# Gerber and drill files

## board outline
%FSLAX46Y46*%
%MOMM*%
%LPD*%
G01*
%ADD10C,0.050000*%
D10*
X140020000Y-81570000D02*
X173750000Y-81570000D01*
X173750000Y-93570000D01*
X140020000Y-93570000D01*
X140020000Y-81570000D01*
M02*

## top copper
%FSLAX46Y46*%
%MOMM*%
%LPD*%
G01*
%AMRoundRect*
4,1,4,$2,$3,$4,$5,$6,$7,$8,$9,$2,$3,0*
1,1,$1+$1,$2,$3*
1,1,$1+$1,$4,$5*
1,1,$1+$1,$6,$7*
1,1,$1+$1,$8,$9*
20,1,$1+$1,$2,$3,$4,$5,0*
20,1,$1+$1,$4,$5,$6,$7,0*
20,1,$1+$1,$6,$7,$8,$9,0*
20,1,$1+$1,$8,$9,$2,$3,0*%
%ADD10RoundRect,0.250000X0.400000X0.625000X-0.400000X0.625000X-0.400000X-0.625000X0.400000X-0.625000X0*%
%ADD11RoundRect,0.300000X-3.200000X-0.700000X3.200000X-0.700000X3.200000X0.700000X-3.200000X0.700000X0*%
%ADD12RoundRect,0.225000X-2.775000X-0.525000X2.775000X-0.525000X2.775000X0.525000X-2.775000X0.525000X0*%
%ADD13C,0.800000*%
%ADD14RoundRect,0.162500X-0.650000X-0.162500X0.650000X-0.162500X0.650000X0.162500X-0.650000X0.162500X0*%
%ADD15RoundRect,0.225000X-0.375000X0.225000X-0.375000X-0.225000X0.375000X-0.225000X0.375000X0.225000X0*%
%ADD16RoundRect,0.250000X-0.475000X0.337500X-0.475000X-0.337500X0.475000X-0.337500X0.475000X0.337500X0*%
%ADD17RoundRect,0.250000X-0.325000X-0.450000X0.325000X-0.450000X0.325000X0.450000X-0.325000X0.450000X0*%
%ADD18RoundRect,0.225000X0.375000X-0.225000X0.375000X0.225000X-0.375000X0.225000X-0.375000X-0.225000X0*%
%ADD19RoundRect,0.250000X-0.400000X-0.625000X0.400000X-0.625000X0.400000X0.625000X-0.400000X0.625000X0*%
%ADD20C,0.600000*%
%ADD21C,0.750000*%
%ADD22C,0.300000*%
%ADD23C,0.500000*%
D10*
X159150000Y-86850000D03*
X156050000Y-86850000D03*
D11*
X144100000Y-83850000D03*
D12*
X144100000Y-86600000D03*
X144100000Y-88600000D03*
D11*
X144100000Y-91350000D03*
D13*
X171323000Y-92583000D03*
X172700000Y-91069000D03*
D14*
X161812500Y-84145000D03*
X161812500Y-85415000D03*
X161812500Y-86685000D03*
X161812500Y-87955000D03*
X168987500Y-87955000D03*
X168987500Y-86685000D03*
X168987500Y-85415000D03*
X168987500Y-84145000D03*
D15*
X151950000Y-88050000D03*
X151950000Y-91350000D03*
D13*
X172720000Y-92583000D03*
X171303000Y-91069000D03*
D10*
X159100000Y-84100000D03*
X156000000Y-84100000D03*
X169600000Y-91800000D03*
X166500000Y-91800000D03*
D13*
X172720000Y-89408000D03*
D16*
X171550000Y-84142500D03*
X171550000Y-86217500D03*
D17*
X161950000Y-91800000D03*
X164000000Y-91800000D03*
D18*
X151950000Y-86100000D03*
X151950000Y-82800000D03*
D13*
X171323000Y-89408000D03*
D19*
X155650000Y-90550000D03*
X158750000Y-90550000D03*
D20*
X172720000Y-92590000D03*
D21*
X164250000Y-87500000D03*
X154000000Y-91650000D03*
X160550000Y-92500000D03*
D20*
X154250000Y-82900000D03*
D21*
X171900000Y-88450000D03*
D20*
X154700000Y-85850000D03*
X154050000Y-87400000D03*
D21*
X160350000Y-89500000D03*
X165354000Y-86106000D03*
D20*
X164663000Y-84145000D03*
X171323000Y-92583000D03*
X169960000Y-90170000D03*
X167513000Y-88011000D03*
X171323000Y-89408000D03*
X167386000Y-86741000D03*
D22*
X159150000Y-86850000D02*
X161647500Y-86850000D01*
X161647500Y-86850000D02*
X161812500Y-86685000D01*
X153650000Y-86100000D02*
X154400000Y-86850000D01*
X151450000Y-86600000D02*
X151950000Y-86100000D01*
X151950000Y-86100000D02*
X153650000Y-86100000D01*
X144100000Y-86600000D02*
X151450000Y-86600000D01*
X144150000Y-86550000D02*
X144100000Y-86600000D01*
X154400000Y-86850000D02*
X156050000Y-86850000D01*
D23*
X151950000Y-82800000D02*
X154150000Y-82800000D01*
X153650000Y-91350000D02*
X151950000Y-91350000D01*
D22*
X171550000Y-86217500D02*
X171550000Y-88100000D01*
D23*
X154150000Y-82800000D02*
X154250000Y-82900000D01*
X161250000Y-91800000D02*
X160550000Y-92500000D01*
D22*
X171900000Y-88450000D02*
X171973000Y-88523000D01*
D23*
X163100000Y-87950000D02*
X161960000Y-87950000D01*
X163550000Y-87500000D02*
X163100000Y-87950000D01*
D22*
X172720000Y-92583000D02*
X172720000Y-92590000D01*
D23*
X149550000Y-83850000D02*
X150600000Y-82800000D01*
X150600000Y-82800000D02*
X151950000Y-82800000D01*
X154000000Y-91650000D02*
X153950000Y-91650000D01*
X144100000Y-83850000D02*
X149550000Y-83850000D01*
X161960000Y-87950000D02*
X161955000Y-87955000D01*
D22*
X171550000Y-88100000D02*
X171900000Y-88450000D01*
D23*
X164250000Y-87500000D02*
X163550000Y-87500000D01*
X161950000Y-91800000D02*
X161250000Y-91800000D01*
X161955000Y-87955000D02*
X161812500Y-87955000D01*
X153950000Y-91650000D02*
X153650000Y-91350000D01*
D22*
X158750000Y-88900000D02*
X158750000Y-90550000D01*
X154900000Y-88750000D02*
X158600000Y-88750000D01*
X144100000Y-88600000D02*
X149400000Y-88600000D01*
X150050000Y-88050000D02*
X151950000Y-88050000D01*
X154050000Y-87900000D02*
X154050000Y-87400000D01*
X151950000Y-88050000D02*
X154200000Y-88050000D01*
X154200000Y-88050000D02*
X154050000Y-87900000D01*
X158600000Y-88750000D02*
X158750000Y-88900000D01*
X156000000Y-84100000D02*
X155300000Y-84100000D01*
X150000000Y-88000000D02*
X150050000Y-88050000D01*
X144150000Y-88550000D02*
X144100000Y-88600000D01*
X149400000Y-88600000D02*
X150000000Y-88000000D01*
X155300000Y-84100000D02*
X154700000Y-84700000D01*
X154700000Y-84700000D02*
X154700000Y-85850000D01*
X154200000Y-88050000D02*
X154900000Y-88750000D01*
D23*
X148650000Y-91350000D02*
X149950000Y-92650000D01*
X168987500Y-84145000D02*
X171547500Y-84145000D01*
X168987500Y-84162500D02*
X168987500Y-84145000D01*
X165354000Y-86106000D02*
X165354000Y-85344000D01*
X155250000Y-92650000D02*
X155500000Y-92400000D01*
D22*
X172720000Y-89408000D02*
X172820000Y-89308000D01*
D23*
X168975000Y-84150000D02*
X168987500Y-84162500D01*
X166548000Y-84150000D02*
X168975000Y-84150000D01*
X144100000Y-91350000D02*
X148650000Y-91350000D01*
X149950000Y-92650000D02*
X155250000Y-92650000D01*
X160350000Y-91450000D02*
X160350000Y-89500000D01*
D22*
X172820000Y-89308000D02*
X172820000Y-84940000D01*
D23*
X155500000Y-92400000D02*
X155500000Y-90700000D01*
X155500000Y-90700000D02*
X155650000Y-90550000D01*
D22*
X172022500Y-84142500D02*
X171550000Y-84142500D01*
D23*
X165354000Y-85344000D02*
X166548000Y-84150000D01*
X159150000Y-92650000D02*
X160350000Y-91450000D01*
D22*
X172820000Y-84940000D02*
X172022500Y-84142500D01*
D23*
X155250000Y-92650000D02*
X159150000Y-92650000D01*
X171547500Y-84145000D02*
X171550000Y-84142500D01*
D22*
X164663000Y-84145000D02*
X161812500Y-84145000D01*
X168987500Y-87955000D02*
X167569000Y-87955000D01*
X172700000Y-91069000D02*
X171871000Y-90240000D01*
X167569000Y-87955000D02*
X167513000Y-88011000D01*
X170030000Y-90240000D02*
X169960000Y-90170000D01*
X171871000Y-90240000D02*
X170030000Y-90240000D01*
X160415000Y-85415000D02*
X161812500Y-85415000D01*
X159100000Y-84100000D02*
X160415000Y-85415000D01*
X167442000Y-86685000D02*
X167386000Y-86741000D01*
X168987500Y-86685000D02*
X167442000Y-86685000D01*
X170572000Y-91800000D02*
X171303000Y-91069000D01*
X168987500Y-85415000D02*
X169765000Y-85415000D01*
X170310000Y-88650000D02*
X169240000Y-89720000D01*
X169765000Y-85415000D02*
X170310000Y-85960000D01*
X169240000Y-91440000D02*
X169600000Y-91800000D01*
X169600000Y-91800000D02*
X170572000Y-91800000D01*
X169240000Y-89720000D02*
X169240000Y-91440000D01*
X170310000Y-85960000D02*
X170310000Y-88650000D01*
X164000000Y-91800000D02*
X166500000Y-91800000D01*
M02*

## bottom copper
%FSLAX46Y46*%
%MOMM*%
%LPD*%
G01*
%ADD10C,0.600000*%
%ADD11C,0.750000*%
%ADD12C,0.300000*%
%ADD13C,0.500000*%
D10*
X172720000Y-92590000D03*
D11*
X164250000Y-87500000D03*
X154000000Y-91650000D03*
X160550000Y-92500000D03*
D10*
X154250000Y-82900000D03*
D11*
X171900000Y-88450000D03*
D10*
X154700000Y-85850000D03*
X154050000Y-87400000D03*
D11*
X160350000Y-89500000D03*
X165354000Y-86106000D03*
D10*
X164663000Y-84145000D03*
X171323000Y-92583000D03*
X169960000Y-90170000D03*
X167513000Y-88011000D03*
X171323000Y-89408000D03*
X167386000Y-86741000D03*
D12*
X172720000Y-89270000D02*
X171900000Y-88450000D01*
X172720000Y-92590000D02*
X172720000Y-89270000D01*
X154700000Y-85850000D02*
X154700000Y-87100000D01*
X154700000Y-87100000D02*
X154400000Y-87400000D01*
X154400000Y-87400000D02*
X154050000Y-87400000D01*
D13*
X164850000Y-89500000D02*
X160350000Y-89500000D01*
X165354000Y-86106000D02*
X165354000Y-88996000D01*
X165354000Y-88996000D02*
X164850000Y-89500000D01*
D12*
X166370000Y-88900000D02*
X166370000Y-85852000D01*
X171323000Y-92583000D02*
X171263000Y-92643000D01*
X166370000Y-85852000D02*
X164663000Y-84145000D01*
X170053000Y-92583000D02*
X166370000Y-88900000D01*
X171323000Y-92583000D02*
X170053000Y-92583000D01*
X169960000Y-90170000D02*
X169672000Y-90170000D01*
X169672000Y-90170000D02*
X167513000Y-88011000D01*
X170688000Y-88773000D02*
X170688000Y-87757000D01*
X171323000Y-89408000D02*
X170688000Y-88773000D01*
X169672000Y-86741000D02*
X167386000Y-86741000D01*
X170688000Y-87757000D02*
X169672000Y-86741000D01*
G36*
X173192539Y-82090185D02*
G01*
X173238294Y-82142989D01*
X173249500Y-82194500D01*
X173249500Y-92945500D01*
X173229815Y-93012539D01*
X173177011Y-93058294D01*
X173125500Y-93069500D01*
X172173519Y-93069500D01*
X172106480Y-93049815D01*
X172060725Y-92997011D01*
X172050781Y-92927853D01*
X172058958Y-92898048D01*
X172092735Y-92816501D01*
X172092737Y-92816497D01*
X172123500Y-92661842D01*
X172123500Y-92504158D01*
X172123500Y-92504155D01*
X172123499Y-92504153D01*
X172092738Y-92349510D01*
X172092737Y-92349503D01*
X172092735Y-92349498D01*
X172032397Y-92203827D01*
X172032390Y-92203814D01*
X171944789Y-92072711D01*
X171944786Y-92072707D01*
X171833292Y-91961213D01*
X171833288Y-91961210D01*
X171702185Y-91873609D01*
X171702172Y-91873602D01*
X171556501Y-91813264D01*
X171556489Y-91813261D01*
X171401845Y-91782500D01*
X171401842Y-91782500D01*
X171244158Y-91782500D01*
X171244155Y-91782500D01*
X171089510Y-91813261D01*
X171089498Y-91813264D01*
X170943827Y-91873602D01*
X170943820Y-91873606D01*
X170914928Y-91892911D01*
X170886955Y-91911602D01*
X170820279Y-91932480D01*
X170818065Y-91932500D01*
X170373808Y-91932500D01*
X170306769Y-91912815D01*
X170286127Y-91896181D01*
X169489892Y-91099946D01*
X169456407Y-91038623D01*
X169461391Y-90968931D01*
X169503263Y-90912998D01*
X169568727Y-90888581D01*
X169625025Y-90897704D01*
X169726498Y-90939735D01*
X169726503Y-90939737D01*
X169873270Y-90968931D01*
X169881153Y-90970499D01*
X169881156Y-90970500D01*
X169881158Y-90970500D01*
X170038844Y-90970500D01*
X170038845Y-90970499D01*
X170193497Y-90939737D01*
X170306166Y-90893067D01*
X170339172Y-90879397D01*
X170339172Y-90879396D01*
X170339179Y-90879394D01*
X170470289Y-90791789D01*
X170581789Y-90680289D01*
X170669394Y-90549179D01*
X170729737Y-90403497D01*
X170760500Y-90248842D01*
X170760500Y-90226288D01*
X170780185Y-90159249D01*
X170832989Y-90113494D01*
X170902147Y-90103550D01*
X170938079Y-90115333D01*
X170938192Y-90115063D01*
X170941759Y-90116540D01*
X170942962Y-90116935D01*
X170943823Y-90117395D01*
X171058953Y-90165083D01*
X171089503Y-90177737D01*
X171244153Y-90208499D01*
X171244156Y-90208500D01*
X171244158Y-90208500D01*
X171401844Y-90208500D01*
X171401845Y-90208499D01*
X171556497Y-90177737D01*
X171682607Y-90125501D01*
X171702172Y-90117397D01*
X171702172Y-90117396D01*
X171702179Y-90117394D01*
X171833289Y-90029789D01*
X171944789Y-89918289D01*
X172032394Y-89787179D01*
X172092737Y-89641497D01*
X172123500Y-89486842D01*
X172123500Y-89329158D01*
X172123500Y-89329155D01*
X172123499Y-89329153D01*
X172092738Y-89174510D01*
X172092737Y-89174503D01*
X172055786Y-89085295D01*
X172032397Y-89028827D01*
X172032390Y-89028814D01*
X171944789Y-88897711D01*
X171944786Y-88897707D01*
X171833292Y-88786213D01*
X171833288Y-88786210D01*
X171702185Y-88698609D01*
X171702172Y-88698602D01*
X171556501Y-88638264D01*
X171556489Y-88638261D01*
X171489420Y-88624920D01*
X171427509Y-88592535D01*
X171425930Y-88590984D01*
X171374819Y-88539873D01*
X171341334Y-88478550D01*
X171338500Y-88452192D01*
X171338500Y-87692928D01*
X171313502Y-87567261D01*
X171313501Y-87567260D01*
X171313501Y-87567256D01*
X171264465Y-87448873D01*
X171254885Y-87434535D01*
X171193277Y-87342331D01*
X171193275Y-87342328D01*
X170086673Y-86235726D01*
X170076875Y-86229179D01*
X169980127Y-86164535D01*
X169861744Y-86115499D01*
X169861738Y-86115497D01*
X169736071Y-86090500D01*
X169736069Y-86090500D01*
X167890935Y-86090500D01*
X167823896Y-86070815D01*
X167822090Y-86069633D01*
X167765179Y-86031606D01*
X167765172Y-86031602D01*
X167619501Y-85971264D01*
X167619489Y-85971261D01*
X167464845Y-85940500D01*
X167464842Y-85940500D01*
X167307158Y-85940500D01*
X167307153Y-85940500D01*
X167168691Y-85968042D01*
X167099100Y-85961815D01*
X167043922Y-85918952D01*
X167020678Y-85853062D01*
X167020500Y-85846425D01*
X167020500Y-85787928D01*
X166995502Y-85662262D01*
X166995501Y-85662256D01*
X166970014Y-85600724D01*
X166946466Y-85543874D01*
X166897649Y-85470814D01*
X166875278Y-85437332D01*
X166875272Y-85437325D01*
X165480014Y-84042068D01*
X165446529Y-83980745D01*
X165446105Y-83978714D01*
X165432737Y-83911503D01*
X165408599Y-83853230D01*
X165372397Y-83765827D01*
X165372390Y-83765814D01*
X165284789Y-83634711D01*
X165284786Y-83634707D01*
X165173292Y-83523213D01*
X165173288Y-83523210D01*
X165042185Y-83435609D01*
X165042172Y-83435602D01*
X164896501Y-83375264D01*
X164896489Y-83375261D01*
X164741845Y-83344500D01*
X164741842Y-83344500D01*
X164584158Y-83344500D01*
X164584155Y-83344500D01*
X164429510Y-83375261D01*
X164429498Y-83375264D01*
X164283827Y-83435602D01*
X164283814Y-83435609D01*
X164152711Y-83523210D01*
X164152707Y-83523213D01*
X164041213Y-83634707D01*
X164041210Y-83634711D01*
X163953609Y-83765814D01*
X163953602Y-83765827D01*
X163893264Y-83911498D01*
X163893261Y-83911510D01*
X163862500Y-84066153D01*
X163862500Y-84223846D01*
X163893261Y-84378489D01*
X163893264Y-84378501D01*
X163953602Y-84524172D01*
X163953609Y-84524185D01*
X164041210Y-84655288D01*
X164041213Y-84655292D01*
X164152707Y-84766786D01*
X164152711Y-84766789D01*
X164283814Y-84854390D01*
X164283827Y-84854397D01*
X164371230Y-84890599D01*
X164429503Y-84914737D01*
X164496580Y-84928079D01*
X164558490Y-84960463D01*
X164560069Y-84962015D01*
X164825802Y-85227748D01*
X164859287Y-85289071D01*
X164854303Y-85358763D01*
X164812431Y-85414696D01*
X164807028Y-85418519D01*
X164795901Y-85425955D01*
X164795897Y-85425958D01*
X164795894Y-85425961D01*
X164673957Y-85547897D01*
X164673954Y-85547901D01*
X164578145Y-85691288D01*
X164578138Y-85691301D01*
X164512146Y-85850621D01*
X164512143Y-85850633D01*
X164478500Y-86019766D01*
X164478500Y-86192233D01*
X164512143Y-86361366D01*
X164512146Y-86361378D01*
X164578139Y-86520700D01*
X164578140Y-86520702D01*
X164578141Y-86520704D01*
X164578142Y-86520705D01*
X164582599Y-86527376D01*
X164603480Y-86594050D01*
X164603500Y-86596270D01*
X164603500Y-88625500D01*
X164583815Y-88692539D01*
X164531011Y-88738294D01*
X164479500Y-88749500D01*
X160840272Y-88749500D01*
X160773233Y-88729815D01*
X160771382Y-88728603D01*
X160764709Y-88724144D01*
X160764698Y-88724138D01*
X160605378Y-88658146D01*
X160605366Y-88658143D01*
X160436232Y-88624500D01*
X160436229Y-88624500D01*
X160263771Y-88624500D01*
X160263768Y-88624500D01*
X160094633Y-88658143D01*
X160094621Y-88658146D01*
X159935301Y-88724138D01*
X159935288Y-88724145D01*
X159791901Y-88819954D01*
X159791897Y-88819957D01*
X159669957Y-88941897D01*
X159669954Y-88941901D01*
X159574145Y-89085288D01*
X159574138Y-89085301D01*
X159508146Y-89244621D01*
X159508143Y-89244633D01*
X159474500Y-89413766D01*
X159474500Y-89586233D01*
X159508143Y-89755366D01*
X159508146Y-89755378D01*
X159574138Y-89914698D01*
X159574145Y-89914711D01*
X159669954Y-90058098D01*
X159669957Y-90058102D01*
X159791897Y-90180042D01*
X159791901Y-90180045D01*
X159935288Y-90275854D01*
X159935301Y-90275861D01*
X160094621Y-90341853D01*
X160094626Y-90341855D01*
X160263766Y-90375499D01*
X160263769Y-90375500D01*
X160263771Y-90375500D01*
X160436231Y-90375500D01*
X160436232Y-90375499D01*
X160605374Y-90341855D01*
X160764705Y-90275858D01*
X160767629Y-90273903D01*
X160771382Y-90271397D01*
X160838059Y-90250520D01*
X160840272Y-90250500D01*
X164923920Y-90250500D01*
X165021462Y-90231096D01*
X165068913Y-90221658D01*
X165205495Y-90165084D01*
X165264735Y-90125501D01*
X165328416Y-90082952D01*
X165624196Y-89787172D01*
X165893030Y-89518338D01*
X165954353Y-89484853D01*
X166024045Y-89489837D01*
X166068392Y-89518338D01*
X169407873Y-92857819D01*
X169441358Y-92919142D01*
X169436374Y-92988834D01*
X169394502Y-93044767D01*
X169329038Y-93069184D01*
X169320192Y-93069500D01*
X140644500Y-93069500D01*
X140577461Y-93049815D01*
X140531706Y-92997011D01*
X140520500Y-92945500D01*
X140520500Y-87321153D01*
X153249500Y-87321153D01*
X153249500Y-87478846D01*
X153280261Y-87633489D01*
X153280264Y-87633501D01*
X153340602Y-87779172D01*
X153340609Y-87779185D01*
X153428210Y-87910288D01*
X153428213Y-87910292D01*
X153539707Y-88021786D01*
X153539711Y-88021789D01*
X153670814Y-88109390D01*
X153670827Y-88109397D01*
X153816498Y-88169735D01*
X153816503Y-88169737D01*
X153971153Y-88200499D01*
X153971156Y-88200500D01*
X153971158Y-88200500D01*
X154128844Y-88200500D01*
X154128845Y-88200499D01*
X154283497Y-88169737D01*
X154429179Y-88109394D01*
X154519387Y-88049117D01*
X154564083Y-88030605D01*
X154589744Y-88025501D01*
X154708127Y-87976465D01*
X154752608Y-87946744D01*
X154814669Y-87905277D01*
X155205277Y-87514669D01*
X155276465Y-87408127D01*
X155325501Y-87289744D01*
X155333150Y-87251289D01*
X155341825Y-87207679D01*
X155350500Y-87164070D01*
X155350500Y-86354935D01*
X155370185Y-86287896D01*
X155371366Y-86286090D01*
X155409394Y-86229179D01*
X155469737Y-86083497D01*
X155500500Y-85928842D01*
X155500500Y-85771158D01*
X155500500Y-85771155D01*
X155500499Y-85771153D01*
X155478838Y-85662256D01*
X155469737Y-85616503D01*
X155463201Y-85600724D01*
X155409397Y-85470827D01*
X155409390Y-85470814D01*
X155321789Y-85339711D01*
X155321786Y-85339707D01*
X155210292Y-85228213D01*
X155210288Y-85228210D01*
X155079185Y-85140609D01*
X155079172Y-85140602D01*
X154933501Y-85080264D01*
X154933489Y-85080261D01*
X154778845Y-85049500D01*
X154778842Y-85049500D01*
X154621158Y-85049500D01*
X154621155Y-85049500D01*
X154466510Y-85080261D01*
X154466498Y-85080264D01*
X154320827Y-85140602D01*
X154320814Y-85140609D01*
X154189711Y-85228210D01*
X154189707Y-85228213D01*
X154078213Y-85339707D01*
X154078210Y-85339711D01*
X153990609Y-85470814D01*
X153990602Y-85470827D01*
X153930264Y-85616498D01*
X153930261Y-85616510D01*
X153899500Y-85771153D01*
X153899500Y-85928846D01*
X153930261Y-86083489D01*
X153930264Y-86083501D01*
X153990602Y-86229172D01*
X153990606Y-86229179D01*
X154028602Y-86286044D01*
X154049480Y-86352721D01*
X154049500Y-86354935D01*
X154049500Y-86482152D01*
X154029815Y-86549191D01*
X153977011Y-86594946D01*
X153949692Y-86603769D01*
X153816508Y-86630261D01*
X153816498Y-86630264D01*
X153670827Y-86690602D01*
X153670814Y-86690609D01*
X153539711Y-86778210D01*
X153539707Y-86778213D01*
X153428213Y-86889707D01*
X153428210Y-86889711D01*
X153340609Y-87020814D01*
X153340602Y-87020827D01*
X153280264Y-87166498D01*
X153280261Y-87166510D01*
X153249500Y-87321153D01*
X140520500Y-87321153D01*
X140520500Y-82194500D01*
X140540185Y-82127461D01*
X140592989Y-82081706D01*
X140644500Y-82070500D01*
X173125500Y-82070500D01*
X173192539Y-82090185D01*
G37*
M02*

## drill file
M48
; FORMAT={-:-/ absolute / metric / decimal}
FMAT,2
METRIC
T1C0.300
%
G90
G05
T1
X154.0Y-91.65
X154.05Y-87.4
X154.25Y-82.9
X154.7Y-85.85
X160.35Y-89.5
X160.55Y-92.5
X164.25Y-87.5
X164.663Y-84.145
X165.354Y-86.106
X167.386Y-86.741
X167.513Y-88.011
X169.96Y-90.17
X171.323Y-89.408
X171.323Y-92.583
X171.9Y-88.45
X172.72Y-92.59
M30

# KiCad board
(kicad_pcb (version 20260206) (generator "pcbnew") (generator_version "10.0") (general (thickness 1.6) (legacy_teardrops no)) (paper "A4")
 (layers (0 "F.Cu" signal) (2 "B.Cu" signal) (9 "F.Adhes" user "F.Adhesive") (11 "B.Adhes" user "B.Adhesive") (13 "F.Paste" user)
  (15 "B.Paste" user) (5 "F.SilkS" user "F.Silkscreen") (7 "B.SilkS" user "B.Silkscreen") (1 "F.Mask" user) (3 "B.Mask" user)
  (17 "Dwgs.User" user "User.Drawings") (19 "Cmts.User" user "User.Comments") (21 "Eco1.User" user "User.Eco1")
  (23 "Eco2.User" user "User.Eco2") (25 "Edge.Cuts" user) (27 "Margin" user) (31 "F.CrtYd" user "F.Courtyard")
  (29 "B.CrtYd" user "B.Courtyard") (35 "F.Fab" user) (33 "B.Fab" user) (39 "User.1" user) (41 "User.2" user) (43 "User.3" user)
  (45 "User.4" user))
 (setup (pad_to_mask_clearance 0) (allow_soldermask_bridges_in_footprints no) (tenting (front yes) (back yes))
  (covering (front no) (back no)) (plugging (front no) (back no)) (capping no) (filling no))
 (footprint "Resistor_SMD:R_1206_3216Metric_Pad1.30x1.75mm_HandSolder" (layer "F.Cu") (at 157.6 86.85 180)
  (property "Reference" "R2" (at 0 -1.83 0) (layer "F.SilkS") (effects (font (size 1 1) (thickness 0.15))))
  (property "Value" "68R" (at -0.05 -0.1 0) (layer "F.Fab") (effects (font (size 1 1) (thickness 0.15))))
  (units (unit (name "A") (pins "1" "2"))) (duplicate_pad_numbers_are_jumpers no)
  (pad "1" smd roundrect (at -1.55 0 180) (size 1.3 1.75) (layers "F.Cu" "F.Mask" "F.Paste") (roundrect_rratio 0.192308) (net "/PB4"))
  (pad "2" smd roundrect (at 1.55 0 180) (size 1.3 1.75) (layers "F.Cu" "F.Mask" "F.Paste") (roundrect_rratio 0.192308) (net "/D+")))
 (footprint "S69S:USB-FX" (layer "F.Cu") (at 144.1 87.6)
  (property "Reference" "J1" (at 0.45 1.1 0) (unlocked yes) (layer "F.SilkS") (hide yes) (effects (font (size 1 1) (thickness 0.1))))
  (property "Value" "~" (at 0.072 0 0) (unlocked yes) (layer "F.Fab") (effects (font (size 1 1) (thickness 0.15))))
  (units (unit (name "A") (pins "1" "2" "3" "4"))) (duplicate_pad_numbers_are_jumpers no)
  (pad "1" smd roundrect (at 0 -3.75) (size 7 2) (layers "F.Cu" "F.Mask" "F.Paste") (roundrect_rratio 0.15) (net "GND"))
  (pad "2" smd roundrect (at 0 -1) (size 6 1.5) (layers "F.Cu" "F.Mask" "F.Paste") (roundrect_rratio 0.15) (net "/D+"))
  (pad "3" smd roundrect (at 0 1) (size 6 1.5) (layers "F.Cu" "F.Mask" "F.Paste") (roundrect_rratio 0.15) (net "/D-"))
  (pad "4" smd roundrect (at 0 3.75) (size 7 2) (layers "F.Cu" "F.Mask" "F.Paste") (roundrect_rratio 0.15) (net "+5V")))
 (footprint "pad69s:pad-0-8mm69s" (layer "F.Cu") (at 171.343 92.573)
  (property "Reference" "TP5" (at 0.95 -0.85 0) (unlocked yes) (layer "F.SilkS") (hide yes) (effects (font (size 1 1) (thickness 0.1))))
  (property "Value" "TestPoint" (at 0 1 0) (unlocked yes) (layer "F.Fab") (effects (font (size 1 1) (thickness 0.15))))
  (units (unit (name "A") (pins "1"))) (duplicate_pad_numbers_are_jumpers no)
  (pad "1" smd circle (at -0.02 0.01) (size 0.8 0.8) (layers "F.Cu" "F.Mask" "F.Paste") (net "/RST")))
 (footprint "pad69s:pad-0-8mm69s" (layer "F.Cu") (at 172.72 91.059)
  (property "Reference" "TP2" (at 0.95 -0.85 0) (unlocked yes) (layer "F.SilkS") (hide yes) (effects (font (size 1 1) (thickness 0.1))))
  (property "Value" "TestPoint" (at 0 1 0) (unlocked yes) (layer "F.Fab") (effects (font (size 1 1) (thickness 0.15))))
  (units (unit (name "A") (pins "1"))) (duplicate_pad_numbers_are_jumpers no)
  (pad "1" smd circle (at -0.02 0.01) (size 0.8 0.8) (layers "F.Cu" "F.Mask" "F.Paste") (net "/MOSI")))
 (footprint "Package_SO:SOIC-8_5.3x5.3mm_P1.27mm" (layer "F.Cu") (at 165.4 86.05)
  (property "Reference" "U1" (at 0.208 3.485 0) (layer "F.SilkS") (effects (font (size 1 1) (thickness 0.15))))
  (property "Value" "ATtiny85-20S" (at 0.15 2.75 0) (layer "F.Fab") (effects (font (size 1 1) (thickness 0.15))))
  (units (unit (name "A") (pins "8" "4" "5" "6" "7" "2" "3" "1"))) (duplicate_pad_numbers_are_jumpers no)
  (pad "1" smd roundrect (at -3.5875 -1.905) (size 1.625 0.65) (layers "F.Cu" "F.Mask" "F.Paste") (roundrect_rratio 0.25) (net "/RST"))
  (pad "2" smd roundrect (at -3.5875 -0.635) (size 1.625 0.65) (layers "F.Cu" "F.Mask" "F.Paste") (roundrect_rratio 0.25) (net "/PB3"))
  (pad "3" smd roundrect (at -3.5875 0.635) (size 1.625 0.65) (layers "F.Cu" "F.Mask" "F.Paste") (roundrect_rratio 0.25) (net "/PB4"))
  (pad "4" smd roundrect (at -3.5875 1.905) (size 1.625 0.65) (layers "F.Cu" "F.Mask" "F.Paste") (roundrect_rratio 0.25) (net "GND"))
  (pad "5" smd roundrect (at 3.5875 1.905) (size 1.625 0.65) (layers "F.Cu" "F.Mask" "F.Paste") (roundrect_rratio 0.25) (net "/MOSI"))
  (pad "6" smd roundrect (at 3.5875 0.635) (size 1.625 0.65) (layers "F.Cu" "F.Mask" "F.Paste") (roundrect_rratio 0.25) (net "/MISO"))
  (pad "7" smd roundrect (at 3.5875 -0.635) (size 1.625 0.65) (layers "F.Cu" "F.Mask" "F.Paste") (roundrect_rratio 0.25) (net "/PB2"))
  (pad "8" smd roundrect (at 3.5875 -1.905) (size 1.625 0.65) (layers "F.Cu" "F.Mask" "F.Paste") (roundrect_rratio 0.25) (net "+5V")))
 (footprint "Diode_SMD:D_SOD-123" (layer "F.Cu") (at 151.95 89.7 -90)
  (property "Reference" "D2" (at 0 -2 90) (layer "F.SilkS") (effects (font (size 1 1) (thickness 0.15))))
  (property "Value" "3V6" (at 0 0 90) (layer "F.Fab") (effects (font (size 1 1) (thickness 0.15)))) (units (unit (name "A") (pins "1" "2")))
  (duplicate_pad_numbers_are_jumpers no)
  (pad "1" smd roundrect (at -1.65 0 270) (size 0.9 1.2) (layers "F.Cu" "F.Mask" "F.Paste") (roundrect_rratio 0.25) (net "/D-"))
  (pad "2" smd roundrect (at 1.65 0 270) (size 0.9 1.2) (layers "F.Cu" "F.Mask" "F.Paste") (roundrect_rratio 0.25) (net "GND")))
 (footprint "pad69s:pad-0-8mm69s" (layer "F.Cu") (at 172.74 92.573)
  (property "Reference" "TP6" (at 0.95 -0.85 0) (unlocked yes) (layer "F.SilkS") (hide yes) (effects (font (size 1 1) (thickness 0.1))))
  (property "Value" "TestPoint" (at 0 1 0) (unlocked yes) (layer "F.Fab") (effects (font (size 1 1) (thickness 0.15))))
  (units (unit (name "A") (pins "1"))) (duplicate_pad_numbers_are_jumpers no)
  (pad "1" smd circle (at -0.02 0.01) (size 0.8 0.8) (layers "F.Cu" "F.Mask" "F.Paste") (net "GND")))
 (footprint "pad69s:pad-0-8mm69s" (layer "F.Cu") (at 171.323 91.059)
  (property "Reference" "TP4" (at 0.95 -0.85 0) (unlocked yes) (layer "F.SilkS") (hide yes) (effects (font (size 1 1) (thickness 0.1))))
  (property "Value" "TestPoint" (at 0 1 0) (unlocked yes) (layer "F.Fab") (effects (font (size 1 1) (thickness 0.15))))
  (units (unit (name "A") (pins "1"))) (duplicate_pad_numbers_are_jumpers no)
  (pad "1" smd circle (at -0.02 0.01) (size 0.8 0.8) (layers "F.Cu" "F.Mask" "F.Paste") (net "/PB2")))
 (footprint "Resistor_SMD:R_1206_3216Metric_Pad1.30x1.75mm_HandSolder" (layer "F.Cu") (at 157.55 84.1 180)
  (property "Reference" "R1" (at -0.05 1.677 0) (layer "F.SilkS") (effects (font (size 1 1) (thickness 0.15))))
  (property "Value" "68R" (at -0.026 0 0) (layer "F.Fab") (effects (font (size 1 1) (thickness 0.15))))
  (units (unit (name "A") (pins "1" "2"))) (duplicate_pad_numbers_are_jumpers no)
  (pad "1" smd roundrect (at -1.55 0 180) (size 1.3 1.75) (layers "F.Cu" "F.Mask" "F.Paste") (roundrect_rratio 0.192308) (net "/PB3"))
  (pad "2" smd roundrect (at 1.55 0 180) (size 1.3 1.75) (layers "F.Cu" "F.Mask" "F.Paste") (roundrect_rratio 0.192308) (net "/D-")))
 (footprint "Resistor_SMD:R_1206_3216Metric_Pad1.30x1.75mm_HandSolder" (layer "F.Cu") (at 168.05 91.8 180)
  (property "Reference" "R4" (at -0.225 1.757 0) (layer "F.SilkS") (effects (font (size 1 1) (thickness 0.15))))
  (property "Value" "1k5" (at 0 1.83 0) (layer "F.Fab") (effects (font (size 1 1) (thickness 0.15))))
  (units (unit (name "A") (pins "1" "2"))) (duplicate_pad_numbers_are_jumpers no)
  (pad "1" smd roundrect (at -1.55 0 180) (size 1.3 1.75) (layers "F.Cu" "F.Mask" "F.Paste") (roundrect_rratio 0.192308) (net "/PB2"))
  (pad "2" smd roundrect (at 1.55 0 180) (size 1.3 1.75) (layers "F.Cu" "F.Mask" "F.Paste") (roundrect_rratio 0.192308) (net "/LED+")))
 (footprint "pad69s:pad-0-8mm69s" (layer "F.Cu") (at 172.74 89.398)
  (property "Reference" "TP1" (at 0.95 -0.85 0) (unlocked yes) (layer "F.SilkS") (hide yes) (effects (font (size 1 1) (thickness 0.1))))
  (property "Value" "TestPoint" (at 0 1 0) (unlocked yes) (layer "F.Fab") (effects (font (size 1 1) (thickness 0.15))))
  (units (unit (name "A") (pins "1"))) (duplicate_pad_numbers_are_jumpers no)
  (pad "1" smd circle (at -0.02 0.01) (size 0.8 0.8) (layers "F.Cu" "F.Mask" "F.Paste") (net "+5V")))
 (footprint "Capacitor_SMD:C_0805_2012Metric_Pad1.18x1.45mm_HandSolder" (layer "F.Cu") (at 171.55 85.18 -90)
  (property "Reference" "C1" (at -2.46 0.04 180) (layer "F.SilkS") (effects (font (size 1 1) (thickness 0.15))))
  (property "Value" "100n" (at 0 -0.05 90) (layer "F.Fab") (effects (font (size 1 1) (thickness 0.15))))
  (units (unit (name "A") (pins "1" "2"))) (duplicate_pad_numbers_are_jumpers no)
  (pad "1" smd roundrect (at -1.0375 0 270) (size 1.175 1.45) (layers "F.Cu" "F.Mask" "F.Paste") (roundrect_rratio 0.212766) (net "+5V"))
  (pad "2" smd roundrect (at 1.0375 0 270) (size 1.175 1.45) (layers "F.Cu" "F.Mask" "F.Paste") (roundrect_rratio 0.212766) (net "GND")))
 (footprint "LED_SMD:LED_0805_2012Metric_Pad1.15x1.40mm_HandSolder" (layer "F.Cu") (at 162.975 91.8)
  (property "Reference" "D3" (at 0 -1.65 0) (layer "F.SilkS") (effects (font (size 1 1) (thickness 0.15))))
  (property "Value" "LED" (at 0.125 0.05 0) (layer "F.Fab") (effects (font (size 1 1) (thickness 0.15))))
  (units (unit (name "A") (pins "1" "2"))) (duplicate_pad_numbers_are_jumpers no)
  (pad "1" smd roundrect (at -1.025 0) (size 1.15 1.4) (layers "F.Cu" "F.Mask" "F.Paste") (roundrect_rratio 0.217391) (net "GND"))
  (pad "2" smd roundrect (at 1.025 0) (size 1.15 1.4) (layers "F.Cu" "F.Mask" "F.Paste") (roundrect_rratio 0.217391) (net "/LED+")))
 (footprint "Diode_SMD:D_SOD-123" (layer "F.Cu") (at 151.95 84.45 90)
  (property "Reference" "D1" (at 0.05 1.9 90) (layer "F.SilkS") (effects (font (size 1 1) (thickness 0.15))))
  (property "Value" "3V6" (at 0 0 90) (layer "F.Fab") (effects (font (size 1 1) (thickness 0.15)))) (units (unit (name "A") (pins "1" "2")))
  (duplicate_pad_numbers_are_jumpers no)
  (pad "1" smd roundrect (at -1.65 0 90) (size 0.9 1.2) (layers "F.Cu" "F.Mask" "F.Paste") (roundrect_rratio 0.25) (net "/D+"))
  (pad "2" smd roundrect (at 1.65 0 90) (size 0.9 1.2) (layers "F.Cu" "F.Mask" "F.Paste") (roundrect_rratio 0.25) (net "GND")))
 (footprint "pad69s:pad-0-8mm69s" (layer "F.Cu") (at 171.343 89.398)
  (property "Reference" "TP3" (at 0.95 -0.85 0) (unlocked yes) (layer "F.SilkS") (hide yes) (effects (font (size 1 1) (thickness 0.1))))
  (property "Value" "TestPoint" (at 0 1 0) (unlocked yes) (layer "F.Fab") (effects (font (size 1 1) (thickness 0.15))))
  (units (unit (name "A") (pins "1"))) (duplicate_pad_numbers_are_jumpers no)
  (pad "1" smd circle (at -0.02 0.01) (size 0.8 0.8) (layers "F.Cu" "F.Mask" "F.Paste") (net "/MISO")))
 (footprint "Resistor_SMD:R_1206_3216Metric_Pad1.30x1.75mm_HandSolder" (layer "F.Cu") (at 157.2 90.55)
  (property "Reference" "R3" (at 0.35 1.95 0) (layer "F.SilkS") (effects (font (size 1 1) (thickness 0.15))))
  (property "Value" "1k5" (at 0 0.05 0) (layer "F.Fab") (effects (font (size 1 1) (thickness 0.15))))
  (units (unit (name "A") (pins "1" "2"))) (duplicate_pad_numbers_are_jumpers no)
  (pad "1" smd roundrect (at -1.55 0) (size 1.3 1.75) (layers "F.Cu" "F.Mask" "F.Paste") (roundrect_rratio 0.192308) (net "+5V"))
  (pad "2" smd roundrect (at 1.55 0) (size 1.3 1.75) (layers "F.Cu" "F.Mask" "F.Paste") (roundrect_rratio 0.192308) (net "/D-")))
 (gr_rect (start 140.02 81.57) (end 173.75 93.57) (stroke (width 0.05) (type solid)) (fill no) (layer "Edge.Cuts"))
 (segment (start 159.15 86.85) (end 161.6475 86.85) (width 0.3) (layer "F.Cu") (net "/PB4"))
 (segment (start 161.6475 86.85) (end 161.8125 86.685) (width 0.3) (layer "F.Cu") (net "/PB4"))
 (segment (start 153.65 86.1) (end 154.4 86.85) (width 0.3) (layer "F.Cu") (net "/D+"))
 (segment (start 151.45 86.6) (end 151.95 86.1) (width 0.3) (layer "F.Cu") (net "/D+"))
 (segment (start 151.95 86.1) (end 153.65 86.1) (width 0.3) (layer "F.Cu") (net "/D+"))
 (segment (start 144.1 86.6) (end 151.45 86.6) (width 0.3) (layer "F.Cu") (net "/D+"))
 (segment (start 144.15 86.55) (end 144.1 86.6) (width 0.3) (layer "F.Cu") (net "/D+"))
 (segment (start 154.4 86.85) (end 156.05 86.85) (width 0.3) (layer "F.Cu") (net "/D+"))
 (segment (start 151.95 82.8) (end 154.15 82.8) (width 0.5) (layer "F.Cu") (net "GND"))
 (segment (start 153.65 91.35) (end 151.95 91.35) (width 0.5) (layer "F.Cu") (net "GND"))
 (segment (start 171.55 86.2175) (end 171.55 88.1) (width 0.3) (layer "F.Cu") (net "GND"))
 (segment (start 154.15 82.8) (end 154.25 82.9) (width 0.5) (layer "F.Cu") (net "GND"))
 (segment (start 161.25 91.8) (end 160.55 92.5) (width 0.5) (layer "F.Cu") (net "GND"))
 (segment (start 171.9 88.45) (end 171.973 88.523) (width 0.3) (layer "F.Cu") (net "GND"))
 (segment (start 163.1 87.95) (end 161.96 87.95) (width 0.5) (layer "F.Cu") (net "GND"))
 (segment (start 163.55 87.5) (end 163.1 87.95) (width 0.5) (layer "F.Cu") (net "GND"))
 (segment (start 172.72 92.583) (end 172.72 92.59) (width 0.3) (layer "F.Cu") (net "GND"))
 (segment (start 149.55 83.85) (end 150.6 82.8) (width 0.5) (layer "F.Cu") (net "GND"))
 (segment (start 150.6 82.8) (end 151.95 82.8) (width 0.5) (layer "F.Cu") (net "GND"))
 (segment (start 154 91.65) (end 153.95 91.65) (width 0.5) (layer "F.Cu") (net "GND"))
 (segment (start 144.1 83.85) (end 149.55 83.85) (width 0.5) (layer "F.Cu") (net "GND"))
 (segment (start 161.96 87.95) (end 161.955 87.955) (width 0.5) (layer "F.Cu") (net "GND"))
 (segment (start 171.55 88.1) (end 171.9 88.45) (width 0.3) (layer "F.Cu") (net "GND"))
 (segment (start 164.25 87.5) (end 163.55 87.5) (width 0.5) (layer "F.Cu") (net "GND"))
 (segment (start 161.95 91.8) (end 161.25 91.8) (width 0.5) (layer "F.Cu") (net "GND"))
 (segment (start 161.955 87.955) (end 161.8125 87.955) (width 0.5) (layer "F.Cu") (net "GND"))
 (segment (start 153.95 91.65) (end 153.65 91.35) (width 0.5) (layer "F.Cu") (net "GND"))
 (via (at 172.72 92.59) (size 0.6) (drill 0.3) (layers "F.Cu" "B.Cu") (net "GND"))
 (via (at 164.25 87.5) (size 0.75) (drill 0.3) (layers "F.Cu" "B.Cu") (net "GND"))
 (via (at 154 91.65) (size 0.75) (drill 0.3) (layers "F.Cu" "B.Cu") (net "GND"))
 (via (at 160.55 92.5) (size 0.75) (drill 0.3) (layers "F.Cu" "B.Cu") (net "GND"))
 (via (at 154.25 82.9) (size 0.6) (drill 0.3) (layers "F.Cu" "B.Cu") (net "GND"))
 (via (at 171.9 88.45) (size 0.75) (drill 0.3) (layers "F.Cu" "B.Cu") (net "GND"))
 (segment (start 172.72 89.27) (end 171.9 88.45) (width 0.3) (layer "B.Cu") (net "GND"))
 (segment (start 172.72 92.59) (end 172.72 89.27) (width 0.3) (layer "B.Cu") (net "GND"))
 (segment (start 158.75 88.9) (end 158.75 90.55) (width 0.3) (layer "F.Cu") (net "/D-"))
 (segment (start 154.9 88.75) (end 158.6 88.75) (width 0.3) (layer "F.Cu") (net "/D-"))
 (segment (start 144.1 88.6) (end 149.4 88.6) (width 0.3) (layer "F.Cu") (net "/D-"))
 (segment (start 150.05 88.05) (end 151.95 88.05) (width 0.3) (layer "F.Cu") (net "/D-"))
 (segment (start 154.05 87.9) (end 154.05 87.4) (width 0.3) (layer "F.Cu") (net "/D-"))
 (segment (start 151.95 88.05) (end 154.2 88.05) (width 0.3) (layer "F.Cu") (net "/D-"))
 (segment (start 154.2 88.05) (end 154.05 87.9) (width 0.3) (layer "F.Cu") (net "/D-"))
 (segment (start 158.6 88.75) (end 158.75 88.9) (width 0.3) (layer "F.Cu") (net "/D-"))
 (segment (start 156 84.1) (end 155.3 84.1) (width 0.3) (layer "F.Cu") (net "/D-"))
 (segment (start 150 88) (end 150.05 88.05) (width 0.3) (layer "F.Cu") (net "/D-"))
 (segment (start 144.15 88.55) (end 144.1 88.6) (width 0.3) (layer "F.Cu") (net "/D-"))
 (segment (start 149.4 88.6) (end 150 88) (width 0.3) (layer "F.Cu") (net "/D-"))
 (segment (start 155.3 84.1) (end 154.7 84.7) (width 0.3) (layer "F.Cu") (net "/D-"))
 (segment (start 154.7 84.7) (end 154.7 85.85) (width 0.3) (layer "F.Cu") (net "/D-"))
 (segment (start 154.2 88.05) (end 154.9 88.75) (width 0.3) (layer "F.Cu") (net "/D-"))
 (via (at 154.7 85.85) (size 0.6) (drill 0.3) (layers "F.Cu" "B.Cu") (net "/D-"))
 (via (at 154.05 87.4) (size 0.6) (drill 0.3) (layers "F.Cu" "B.Cu") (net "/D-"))
 (segment (start 154.7 85.85) (end 154.7 87.1) (width 0.3) (layer "B.Cu") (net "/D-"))
 (segment (start 154.7 87.1) (end 154.4 87.4) (width 0.3) (layer "B.Cu") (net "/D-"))
 (segment (start 154.4 87.4) (end 154.05 87.4) (width 0.3) (layer "B.Cu") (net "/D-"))
 (segment (start 148.65 91.35) (end 149.95 92.65) (width 0.5) (layer "F.Cu") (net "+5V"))
 (segment (start 168.9875 84.145) (end 171.5475 84.145) (width 0.5) (layer "F.Cu") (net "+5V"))
 (segment (start 168.9875 84.1625) (end 168.9875 84.145) (width 0.5) (layer "F.Cu") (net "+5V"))
 (segment (start 165.354 86.106) (end 165.354 85.344) (width 0.5) (layer "F.Cu") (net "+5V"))
 (segment (start 155.25 92.65) (end 155.5 92.4) (width 0.5) (layer "F.Cu") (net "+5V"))
 (segment (start 172.72 89.408) (end 172.82 89.308) (width 0.3) (layer "F.Cu") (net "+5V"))
 (segment (start 168.975 84.15) (end 168.9875 84.1625) (width 0.5) (layer "F.Cu") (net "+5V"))
 (segment (start 166.548 84.15) (end 168.975 84.15) (width 0.5) (layer "F.Cu") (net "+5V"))
 (segment (start 144.1 91.35) (end 148.65 91.35) (width 0.5) (layer "F.Cu") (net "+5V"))
 (segment (start 149.95 92.65) (end 155.25 92.65) (width 0.5) (layer "F.Cu") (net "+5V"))
 (segment (start 160.35 91.45) (end 160.35 89.5) (width 0.5) (layer "F.Cu") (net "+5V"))
 (segment (start 172.82 89.308) (end 172.82 84.94) (width 0.3) (layer "F.Cu") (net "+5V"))
 (segment (start 155.5 92.4) (end 155.5 90.7) (width 0.5) (layer "F.Cu") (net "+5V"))
 (segment (start 155.5 90.7) (end 155.65 90.55) (width 0.5) (layer "F.Cu") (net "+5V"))
 (segment (start 172.0225 84.1425) (end 171.55 84.1425) (width 0.3) (layer "F.Cu") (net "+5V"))
 (segment (start 165.354 85.344) (end 166.548 84.15) (width 0.5) (layer "F.Cu") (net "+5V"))
 (segment (start 159.15 92.65) (end 160.35 91.45) (width 0.5) (layer "F.Cu") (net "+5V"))
 (segment (start 172.82 84.94) (end 172.0225 84.1425) (width 0.3) (layer "F.Cu") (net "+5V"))
 (segment (start 155.25 92.65) (end 159.15 92.65) (width 0.5) (layer "F.Cu") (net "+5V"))
 (segment (start 171.5475 84.145) (end 171.55 84.1425) (width 0.5) (layer "F.Cu") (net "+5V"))
 (via (at 160.35 89.5) (size 0.75) (drill 0.3) (layers "F.Cu" "B.Cu") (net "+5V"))
 (via (at 165.354 86.106) (size 0.75) (drill 0.3) (layers "F.Cu" "B.Cu") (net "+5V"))
 (segment (start 164.85 89.5) (end 160.35 89.5) (width 0.5) (layer "B.Cu") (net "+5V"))
 (segment (start 165.354 86.106) (end 165.354 88.996) (width 0.5) (layer "B.Cu") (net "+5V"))
 (segment (start 165.354 88.996) (end 164.85 89.5) (width 0.5) (layer "B.Cu") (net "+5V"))
 (segment (start 164.663 84.145) (end 161.8125 84.145) (width 0.3) (layer "F.Cu") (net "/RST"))
 (via (at 164.663 84.145) (size 0.6) (drill 0.3) (layers "F.Cu" "B.Cu") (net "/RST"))
 (via (at 171.323 92.583) (size 0.6) (drill 0.3) (layers "F.Cu" "B.Cu") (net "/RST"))
 (segment (start 166.37 88.9) (end 166.37 85.852) (width 0.3) (layer "B.Cu") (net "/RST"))
 (segment (start 171.323 92.583) (end 171.263 92.643) (width 0.3) (layer "B.Cu") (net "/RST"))
 (segment (start 166.37 85.852) (end 164.663 84.145) (width 0.3) (layer "B.Cu") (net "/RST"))
 (segment (start 170.053 92.583) (end 166.37 88.9) (width 0.3) (layer "B.Cu") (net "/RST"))
 (segment (start 171.323 92.583) (end 170.053 92.583) (width 0.3) (layer "B.Cu") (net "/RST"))
 (segment (start 168.9875 87.955) (end 167.569 87.955) (width 0.3) (layer "F.Cu") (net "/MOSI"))
 (segment (start 172.7 91.069) (end 171.871 90.24) (width 0.3) (layer "F.Cu") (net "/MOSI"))
 (segment (start 167.569 87.955) (end 167.513 88.011) (width 0.3) (layer "F.Cu") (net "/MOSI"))
 (segment (start 170.03 90.24) (end 169.96 90.17) (width 0.3) (layer "F.Cu") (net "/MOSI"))
 (segment (start 171.871 90.24) (end 170.03 90.24) (width 0.3) (layer "F.Cu") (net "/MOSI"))
 (via (at 169.96 90.17) (size 0.6) (drill 0.3) (layers "F.Cu" "B.Cu") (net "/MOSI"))
 (via (at 167.513 88.011) (size 0.6) (drill 0.3) (layers "F.Cu" "B.Cu") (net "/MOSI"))
 (segment (start 169.96 90.17) (end 169.672 90.17) (width 0.3) (layer "B.Cu") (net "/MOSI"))
 (segment (start 169.672 90.17) (end 167.513 88.011) (width 0.3) (layer "B.Cu") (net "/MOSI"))
 (segment (start 160.415 85.415) (end 161.8125 85.415) (width 0.3) (layer "F.Cu") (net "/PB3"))
 (segment (start 159.1 84.1) (end 160.415 85.415) (width 0.3) (layer "F.Cu") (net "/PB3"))
 (segment (start 167.442 86.685) (end 167.386 86.741) (width 0.3) (layer "F.Cu") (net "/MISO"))
 (segment (start 168.9875 86.685) (end 167.442 86.685) (width 0.3) (layer "F.Cu") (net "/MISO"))
 (via (at 171.323 89.408) (size 0.6) (drill 0.3) (layers "F.Cu" "B.Cu") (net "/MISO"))
 (via (at 167.386 86.741) (size 0.6) (drill 0.3) (layers "F.Cu" "B.Cu") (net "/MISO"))
 (segment (start 170.688 88.773) (end 170.688 87.757) (width 0.3) (layer "B.Cu") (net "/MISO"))
 (segment (start 171.323 89.408) (end 170.688 88.773) (width 0.3) (layer "B.Cu") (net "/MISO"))
 (segment (start 169.672 86.741) (end 167.386 86.741) (width 0.3) (layer "B.Cu") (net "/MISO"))
 (segment (start 170.688 87.757) (end 169.672 86.741) (width 0.3) (layer "B.Cu") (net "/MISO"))
 (segment (start 170.572 91.8) (end 171.303 91.069) (width 0.3) (layer "F.Cu") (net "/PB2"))
 (segment (start 168.9875 85.415) (end 169.765 85.415) (width 0.3) (layer "F.Cu") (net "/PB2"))
 (segment (start 170.31 88.65) (end 169.24 89.72) (width 0.3) (layer "F.Cu") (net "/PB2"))
 (segment (start 169.765 85.415) (end 170.31 85.96) (width 0.3) (layer "F.Cu") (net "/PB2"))
 (segment (start 169.24 91.44) (end 169.6 91.8) (width 0.3) (layer "F.Cu") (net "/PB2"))
 (segment (start 169.6 91.8) (end 170.572 91.8) (width 0.3) (layer "F.Cu") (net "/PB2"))
 (segment (start 169.24 89.72) (end 169.24 91.44) (width 0.3) (layer "F.Cu") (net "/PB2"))
 (segment (start 170.31 85.96) (end 170.31 88.65) (width 0.3) (layer "F.Cu") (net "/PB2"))
 (segment (start 164 91.8) (end 166.5 91.8) (width 0.3) (layer "F.Cu") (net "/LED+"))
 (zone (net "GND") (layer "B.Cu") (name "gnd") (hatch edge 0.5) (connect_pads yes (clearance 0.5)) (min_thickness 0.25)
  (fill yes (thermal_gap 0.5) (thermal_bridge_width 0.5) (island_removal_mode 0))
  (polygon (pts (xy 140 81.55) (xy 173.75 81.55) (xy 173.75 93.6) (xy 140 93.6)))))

